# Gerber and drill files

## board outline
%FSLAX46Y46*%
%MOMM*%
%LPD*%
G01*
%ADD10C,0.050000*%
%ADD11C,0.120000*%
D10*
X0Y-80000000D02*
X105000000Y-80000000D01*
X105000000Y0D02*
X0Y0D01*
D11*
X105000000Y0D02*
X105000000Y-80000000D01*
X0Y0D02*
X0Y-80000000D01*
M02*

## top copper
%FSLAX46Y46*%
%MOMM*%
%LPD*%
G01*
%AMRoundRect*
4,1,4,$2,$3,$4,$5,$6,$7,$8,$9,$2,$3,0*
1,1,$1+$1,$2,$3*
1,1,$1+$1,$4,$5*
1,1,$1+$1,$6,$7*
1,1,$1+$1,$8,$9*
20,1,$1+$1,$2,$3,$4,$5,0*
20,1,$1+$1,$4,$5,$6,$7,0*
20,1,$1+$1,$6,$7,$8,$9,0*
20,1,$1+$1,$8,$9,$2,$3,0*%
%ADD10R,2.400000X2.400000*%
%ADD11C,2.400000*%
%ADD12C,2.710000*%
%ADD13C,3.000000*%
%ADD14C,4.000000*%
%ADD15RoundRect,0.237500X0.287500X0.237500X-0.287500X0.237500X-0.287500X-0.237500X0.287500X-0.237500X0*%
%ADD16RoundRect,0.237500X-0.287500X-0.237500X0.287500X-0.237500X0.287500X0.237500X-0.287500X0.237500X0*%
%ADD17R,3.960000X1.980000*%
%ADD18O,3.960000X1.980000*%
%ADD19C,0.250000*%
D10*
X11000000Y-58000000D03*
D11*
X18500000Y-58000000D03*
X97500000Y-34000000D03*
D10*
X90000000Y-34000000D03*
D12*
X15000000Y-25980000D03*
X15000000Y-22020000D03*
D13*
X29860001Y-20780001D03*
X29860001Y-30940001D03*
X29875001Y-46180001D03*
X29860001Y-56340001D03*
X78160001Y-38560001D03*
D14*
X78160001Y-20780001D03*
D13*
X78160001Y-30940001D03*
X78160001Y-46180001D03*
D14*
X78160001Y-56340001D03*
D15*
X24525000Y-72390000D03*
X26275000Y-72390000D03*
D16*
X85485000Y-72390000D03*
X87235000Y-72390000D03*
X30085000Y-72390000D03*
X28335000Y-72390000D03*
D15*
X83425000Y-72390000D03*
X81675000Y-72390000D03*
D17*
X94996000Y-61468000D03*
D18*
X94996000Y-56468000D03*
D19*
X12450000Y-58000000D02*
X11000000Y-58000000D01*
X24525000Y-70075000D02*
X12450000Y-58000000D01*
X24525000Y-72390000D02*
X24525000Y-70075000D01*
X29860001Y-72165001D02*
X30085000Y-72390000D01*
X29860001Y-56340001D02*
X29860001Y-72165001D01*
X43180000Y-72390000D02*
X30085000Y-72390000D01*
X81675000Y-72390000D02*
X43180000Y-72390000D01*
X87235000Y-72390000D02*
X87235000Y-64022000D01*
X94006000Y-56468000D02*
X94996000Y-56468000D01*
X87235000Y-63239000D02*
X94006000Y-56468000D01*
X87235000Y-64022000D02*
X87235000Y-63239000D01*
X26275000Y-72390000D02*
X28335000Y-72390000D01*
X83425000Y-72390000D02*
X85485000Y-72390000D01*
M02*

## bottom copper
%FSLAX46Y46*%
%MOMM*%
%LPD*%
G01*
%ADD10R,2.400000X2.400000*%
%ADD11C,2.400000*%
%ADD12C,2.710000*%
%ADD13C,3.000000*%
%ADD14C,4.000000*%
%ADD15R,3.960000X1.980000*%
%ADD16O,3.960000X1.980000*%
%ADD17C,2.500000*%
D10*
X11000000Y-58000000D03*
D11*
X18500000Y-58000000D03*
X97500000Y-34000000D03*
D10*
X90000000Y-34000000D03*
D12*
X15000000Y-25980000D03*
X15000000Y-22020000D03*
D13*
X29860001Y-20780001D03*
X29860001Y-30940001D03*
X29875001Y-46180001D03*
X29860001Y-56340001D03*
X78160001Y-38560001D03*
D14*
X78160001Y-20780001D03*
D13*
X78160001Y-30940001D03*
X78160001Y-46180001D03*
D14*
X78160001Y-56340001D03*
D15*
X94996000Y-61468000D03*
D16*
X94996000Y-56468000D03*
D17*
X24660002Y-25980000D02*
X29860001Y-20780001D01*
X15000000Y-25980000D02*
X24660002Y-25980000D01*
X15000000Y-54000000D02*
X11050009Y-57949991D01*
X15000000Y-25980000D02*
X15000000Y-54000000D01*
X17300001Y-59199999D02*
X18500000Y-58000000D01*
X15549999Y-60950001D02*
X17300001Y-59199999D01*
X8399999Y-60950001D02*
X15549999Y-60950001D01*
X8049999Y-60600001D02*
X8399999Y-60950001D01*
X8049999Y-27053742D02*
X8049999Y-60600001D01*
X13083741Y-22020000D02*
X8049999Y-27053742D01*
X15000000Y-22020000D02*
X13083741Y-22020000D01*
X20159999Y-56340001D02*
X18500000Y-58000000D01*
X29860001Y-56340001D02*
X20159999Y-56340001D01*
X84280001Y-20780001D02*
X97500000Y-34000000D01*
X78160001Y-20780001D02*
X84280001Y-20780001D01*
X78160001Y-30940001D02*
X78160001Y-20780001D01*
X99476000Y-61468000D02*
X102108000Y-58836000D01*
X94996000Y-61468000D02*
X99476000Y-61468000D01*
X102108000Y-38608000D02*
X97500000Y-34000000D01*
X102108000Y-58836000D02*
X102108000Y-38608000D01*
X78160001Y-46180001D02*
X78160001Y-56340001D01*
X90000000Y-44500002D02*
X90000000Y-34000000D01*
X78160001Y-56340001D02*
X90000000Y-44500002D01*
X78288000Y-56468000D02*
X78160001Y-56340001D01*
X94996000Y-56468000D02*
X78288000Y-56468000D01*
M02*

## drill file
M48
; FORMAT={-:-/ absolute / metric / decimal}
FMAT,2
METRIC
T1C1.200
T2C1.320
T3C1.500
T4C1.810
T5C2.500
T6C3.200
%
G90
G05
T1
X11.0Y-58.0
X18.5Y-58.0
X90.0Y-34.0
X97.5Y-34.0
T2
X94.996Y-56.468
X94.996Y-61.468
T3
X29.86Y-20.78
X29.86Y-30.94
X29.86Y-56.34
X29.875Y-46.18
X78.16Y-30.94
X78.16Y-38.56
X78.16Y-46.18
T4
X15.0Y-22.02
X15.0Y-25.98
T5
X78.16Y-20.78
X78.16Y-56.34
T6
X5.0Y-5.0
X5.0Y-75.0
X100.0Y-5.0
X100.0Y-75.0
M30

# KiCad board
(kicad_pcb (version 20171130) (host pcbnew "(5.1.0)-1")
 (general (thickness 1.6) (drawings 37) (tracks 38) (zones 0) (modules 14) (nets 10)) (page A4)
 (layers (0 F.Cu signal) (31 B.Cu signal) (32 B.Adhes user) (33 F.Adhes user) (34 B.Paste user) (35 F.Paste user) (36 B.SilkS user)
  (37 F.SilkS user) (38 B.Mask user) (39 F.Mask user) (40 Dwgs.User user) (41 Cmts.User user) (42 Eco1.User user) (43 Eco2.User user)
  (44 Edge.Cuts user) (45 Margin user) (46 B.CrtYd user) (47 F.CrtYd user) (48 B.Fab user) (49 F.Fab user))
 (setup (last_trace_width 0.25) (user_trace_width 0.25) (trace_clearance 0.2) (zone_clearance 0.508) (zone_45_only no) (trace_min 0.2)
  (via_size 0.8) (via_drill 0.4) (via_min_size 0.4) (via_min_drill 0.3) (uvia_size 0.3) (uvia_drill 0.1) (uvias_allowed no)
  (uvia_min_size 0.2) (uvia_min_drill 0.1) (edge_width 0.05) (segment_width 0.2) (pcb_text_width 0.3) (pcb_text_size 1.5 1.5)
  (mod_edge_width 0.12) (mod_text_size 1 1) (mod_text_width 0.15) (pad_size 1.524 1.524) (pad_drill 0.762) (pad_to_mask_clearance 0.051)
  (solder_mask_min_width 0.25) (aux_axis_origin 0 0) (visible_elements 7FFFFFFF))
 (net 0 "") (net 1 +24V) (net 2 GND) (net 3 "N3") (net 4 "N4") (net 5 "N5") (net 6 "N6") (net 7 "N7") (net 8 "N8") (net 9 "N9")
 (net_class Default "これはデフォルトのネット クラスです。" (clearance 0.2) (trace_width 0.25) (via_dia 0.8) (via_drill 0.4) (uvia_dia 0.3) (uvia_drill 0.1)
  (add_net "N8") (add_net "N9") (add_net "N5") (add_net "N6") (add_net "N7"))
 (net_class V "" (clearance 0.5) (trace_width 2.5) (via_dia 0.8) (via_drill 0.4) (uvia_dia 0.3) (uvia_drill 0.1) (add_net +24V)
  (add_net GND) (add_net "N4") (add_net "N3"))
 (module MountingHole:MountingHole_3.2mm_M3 (layer F.Cu) (at 5 5)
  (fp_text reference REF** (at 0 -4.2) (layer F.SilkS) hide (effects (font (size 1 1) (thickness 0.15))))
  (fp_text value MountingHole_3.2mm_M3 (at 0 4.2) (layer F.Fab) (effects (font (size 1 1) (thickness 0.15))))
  (pad 1 np_thru_hole circle (at 0 0) (size 3.2 3.2) (drill 3.2) (layers *.Cu *.Mask)))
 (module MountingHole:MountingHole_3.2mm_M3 (layer F.Cu) (at 5 75)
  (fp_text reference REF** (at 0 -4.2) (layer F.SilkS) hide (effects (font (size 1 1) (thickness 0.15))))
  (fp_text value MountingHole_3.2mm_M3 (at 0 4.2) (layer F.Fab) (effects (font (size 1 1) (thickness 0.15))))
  (pad 1 np_thru_hole circle (at 0 0) (size 3.2 3.2) (drill 3.2) (layers *.Cu *.Mask)))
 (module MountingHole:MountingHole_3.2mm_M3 (layer F.Cu) (at 100 75)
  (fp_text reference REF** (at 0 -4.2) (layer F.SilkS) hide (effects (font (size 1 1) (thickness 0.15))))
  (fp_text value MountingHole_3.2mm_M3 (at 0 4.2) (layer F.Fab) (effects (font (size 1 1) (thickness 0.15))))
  (pad 1 np_thru_hole circle (at 0 0) (size 3.2 3.2) (drill 3.2) (layers *.Cu *.Mask)))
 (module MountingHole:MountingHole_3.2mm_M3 (layer F.Cu) (at 100 5)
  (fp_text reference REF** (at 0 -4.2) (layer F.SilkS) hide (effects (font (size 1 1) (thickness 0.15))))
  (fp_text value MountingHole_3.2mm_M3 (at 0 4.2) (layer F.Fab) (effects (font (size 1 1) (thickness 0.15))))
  (pad 1 np_thru_hole circle (at 0 0) (size 3.2 3.2) (drill 3.2) (layers *.Cu *.Mask)))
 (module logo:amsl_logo (layer F.Cu) (at 13 13)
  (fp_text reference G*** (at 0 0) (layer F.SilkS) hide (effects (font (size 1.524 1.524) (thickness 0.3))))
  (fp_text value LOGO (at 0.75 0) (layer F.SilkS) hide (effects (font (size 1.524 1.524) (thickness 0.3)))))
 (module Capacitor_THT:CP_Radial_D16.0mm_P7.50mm (layer F.Cu) (at 11 58)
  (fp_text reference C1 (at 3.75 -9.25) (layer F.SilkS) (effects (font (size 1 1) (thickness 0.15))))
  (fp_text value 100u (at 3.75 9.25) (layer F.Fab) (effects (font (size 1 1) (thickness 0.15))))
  (pad 1 thru_hole rect (at 0 0) (size 2.4 2.4) (drill 1.2) (layers *.Cu *.Mask) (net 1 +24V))
  (pad 2 thru_hole circle (at 7.5 0) (size 2.4 2.4) (drill 1.2) (layers *.Cu *.Mask) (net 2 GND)))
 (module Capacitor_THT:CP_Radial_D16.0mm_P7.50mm (layer F.Cu) (at 90 34)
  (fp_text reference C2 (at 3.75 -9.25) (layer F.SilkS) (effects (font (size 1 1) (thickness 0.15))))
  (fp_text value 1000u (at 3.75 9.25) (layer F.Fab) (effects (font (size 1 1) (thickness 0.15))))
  (pad 2 thru_hole circle (at 7.5 0) (size 2.4 2.4) (drill 1.2) (layers *.Cu *.Mask) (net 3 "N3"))
  (pad 1 thru_hole rect (at 0 0) (size 2.4 2.4) (drill 1.2) (layers *.Cu *.Mask) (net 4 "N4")))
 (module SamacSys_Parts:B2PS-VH (layer F.Cu) (at 15 24 270)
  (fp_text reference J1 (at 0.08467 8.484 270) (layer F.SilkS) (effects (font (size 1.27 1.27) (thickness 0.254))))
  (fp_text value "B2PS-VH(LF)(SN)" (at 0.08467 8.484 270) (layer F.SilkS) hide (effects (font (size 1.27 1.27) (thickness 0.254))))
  (pad 2 thru_hole circle (at 1.98 0 270) (size 2.71 2.71) (drill 1.81) (layers *.Cu *.Mask) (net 1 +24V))
  (pad 1 thru_hole circle (at -1.98 0 270) (size 2.71 2.71) (drill 1.81) (layers *.Cu *.Mask) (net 2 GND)))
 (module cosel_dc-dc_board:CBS (layer F.Cu) (at 54.010001 38.560001)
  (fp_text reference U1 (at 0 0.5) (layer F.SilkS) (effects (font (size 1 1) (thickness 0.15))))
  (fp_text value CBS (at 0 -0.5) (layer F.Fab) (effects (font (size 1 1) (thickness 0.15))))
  (pad 1 thru_hole circle (at -24.15 -17.78) (size 3 3) (drill 1.5) (layers *.Cu *.Mask) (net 1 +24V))
  (pad 2 thru_hole circle (at -24.15 -7.62) (size 3 3) (drill 1.5) (layers *.Cu *.Mask) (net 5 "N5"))
  (pad 3 thru_hole circle (at -24.135 7.62) (size 3 3) (drill 1.5) (layers *.Cu *.Mask) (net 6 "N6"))
  (pad 4 thru_hole circle (at -24.15 17.78) (size 3 3) (drill 1.5) (layers *.Cu *.Mask) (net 2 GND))
  (pad 7 thru_hole circle (at 24.15 0) (size 3 3) (drill 1.5) (layers *.Cu *.Mask) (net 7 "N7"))
  (pad 5 thru_hole circle (at 24.15 -17.78) (size 4 4) (drill 2.5) (layers *.Cu *.Mask) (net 3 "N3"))
  (pad 6 thru_hole circle (at 24.15 -7.62) (size 3 3) (drill 1.5) (layers *.Cu *.Mask) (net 3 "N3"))
  (pad 8 thru_hole circle (at 24.15 7.62) (size 3 3) (drill 1.5) (layers *.Cu *.Mask) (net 4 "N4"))
  (pad 9 thru_hole circle (at 24.15 17.78) (size 4 4) (drill 2.5) (layers *.Cu *.Mask) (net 4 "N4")))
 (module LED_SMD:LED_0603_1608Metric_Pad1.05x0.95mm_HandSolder (layer F.Cu) (at 25.4 72.39 180)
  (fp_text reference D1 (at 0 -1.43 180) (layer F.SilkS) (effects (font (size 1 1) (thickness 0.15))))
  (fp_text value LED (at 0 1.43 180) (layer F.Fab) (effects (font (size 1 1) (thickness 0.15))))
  (pad 2 smd roundrect (at 0.875 0 180) (size 1.05 0.95) (layers F.Cu F.Paste F.Mask) (roundrect_rratio 0.25) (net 1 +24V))
  (pad 1 smd roundrect (at -0.875 0 180) (size 1.05 0.95) (layers F.Cu F.Paste F.Mask) (roundrect_rratio 0.25) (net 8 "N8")))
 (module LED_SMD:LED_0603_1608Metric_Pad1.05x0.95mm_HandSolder (layer F.Cu) (at 86.36 72.39)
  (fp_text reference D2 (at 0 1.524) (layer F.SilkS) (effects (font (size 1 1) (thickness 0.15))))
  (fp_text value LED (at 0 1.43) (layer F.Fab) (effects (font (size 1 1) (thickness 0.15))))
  (pad 1 smd roundrect (at -0.875 0) (size 1.05 0.95) (layers F.Cu F.Paste F.Mask) (roundrect_rratio 0.25) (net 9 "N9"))
  (pad 2 smd roundrect (at 0.875 0) (size 1.05 0.95) (layers F.Cu F.Paste F.Mask) (roundrect_rratio 0.25) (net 4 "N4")))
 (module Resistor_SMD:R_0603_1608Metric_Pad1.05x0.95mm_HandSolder (layer F.Cu) (at 29.21 72.39)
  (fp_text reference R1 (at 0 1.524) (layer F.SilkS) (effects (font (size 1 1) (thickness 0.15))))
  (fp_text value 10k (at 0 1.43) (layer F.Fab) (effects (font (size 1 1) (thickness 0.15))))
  (pad 2 smd roundrect (at 0.875 0) (size 1.05 0.95) (layers F.Cu F.Paste F.Mask) (roundrect_rratio 0.25) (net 2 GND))
  (pad 1 smd roundrect (at -0.875 0) (size 1.05 0.95) (layers F.Cu F.Paste F.Mask) (roundrect_rratio 0.25) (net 8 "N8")))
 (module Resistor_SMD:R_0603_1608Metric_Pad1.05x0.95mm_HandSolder (layer F.Cu) (at 82.55 72.39 180)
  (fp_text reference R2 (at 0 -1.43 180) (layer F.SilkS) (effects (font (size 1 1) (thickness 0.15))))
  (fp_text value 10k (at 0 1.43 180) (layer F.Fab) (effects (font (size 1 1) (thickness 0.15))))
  (pad 1 smd roundrect (at -0.875 0 180) (size 1.05 0.95) (layers F.Cu F.Paste F.Mask) (roundrect_rratio 0.25) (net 9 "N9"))
  (pad 2 smd roundrect (at 0.875 0 180) (size 1.05 0.95) (layers F.Cu F.Paste F.Mask) (roundrect_rratio 0.25) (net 2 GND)))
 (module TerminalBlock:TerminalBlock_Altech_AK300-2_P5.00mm (layer F.Cu) (at 94.996 61.468 90)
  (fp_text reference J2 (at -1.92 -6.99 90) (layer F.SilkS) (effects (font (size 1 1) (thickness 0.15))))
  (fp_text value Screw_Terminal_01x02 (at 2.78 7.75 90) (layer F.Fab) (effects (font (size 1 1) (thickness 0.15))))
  (pad 1 thru_hole rect (at 0 0 90) (size 1.98 3.96) (drill 1.32) (layers *.Cu *.Mask) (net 3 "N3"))
  (pad 2 thru_hole oval (at 5 0 90) (size 1.98 3.96) (drill 1.32) (layers *.Cu *.Mask) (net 4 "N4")))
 (gr_line (start 0 80) (end 105 80) (layer Edge.Cuts) (width 0.05))
 (gr_line (start 105 0) (end 0 0) (layer Edge.Cuts) (width 0.05))
 (gr_line (start 105 0) (end 105 80) (layer Edge.Cuts) (width 0.12))
 (gr_line (start 0 0) (end 0 80) (layer Edge.Cuts) (width 0.12))
 (segment (start 24.660002 25.98) (end 29.860001 20.780001) (width 2.5) (layer B.Cu) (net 1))
 (segment (start 15 25.98) (end 24.660002 25.98) (width 2.5) (layer B.Cu) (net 1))
 (segment (start 15 54) (end 11.050009 57.949991) (width 2.5) (layer B.Cu) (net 1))
 (segment (start 15 25.98) (end 15 54) (width 2.5) (layer B.Cu) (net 1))
 (segment (start 12.45 58) (end 11 58) (width 0.25) (layer F.Cu) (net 1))
 (segment (start 24.525 70.075) (end 12.45 58) (width 0.25) (layer F.Cu) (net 1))
 (segment (start 24.525 72.39) (end 24.525 70.075) (width 0.25) (layer F.Cu) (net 1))
 (segment (start 17.300001 59.199999) (end 18.5 58) (width 2.5) (layer B.Cu) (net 2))
 (segment (start 15.549999 60.950001) (end 17.300001 59.199999) (width 2.5) (layer B.Cu) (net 2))
 (segment (start 8.399999 60.950001) (end 15.549999 60.950001) (width 2.5) (layer B.Cu) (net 2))
 (segment (start 8.049999 60.600001) (end 8.399999 60.950001) (width 2.5) (layer B.Cu) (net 2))
 (segment (start 8.049999 27.053742) (end 8.049999 60.600001) (width 2.5) (layer B.Cu) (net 2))
 (segment (start 13.083741 22.02) (end 8.049999 27.053742) (width 2.5) (layer B.Cu) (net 2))
 (segment (start 15 22.02) (end 13.083741 22.02) (width 2.5) (layer B.Cu) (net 2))
 (segment (start 20.159999 56.340001) (end 18.5 58) (width 2.5) (layer B.Cu) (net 2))
 (segment (start 29.860001 56.340001) (end 20.159999 56.340001) (width 2.5) (layer B.Cu) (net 2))
 (segment (start 29.860001 72.165001) (end 30.085 72.39) (width 0.25) (layer F.Cu) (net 2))
 (segment (start 29.860001 56.340001) (end 29.860001 72.165001) (width 0.25) (layer F.Cu) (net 2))
 (segment (start 43.18 72.39) (end 30.085 72.39) (width 0.25) (layer F.Cu) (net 2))
 (segment (start 81.675 72.39) (end 43.18 72.39) (width 0.25) (layer F.Cu) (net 2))
 (segment (start 84.280001 20.780001) (end 97.5 34) (width 2.5) (layer B.Cu) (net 3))
 (segment (start 78.160001 20.780001) (end 84.280001 20.780001) (width 2.5) (layer B.Cu) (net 3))
 (segment (start 78.160001 30.940001) (end 78.160001 20.780001) (width 2.5) (layer B.Cu) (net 3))
 (segment (start 99.476 61.468) (end 102.108 58.836) (width 2.5) (layer B.Cu) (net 3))
 (segment (start 94.996 61.468) (end 99.476 61.468) (width 2.5) (layer B.Cu) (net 3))
 (segment (start 102.108 38.608) (end 97.5 34) (width 2.5) (layer B.Cu) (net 3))
 (segment (start 102.108 58.836) (end 102.108 38.608) (width 2.5) (layer B.Cu) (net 3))
 (segment (start 78.160001 46.180001) (end 78.160001 56.340001) (width 2.5) (layer B.Cu) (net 4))
 (segment (start 90 44.500002) (end 90 34) (width 2.5) (layer B.Cu) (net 4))
 (segment (start 78.160001 56.340001) (end 90 44.500002) (width 2.5) (layer B.Cu) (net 4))
 (segment (start 87.235 72.39) (end 87.235 64.022) (width 0.25) (layer F.Cu) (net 4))
 (segment (start 78.288 56.468) (end 78.160001 56.340001) (width 2.5) (layer B.Cu) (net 4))
 (segment (start 94.996 56.468) (end 78.288 56.468) (width 2.5) (layer B.Cu) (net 4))
 (segment (start 94.006 56.468) (end 94.996 56.468) (width 0.25) (layer F.Cu) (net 4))
 (segment (start 87.235 63.239) (end 94.006 56.468) (width 0.25) (layer F.Cu) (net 4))
 (segment (start 87.235 64.022) (end 87.235 63.239) (width 0.25) (layer F.Cu) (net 4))
 (segment (start 26.275 72.39) (end 28.335 72.39) (width 0.25) (layer F.Cu) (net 8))
 (segment (start 83.425 72.39) (end 85.485 72.39) (width 0.25) (layer F.Cu) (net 9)))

